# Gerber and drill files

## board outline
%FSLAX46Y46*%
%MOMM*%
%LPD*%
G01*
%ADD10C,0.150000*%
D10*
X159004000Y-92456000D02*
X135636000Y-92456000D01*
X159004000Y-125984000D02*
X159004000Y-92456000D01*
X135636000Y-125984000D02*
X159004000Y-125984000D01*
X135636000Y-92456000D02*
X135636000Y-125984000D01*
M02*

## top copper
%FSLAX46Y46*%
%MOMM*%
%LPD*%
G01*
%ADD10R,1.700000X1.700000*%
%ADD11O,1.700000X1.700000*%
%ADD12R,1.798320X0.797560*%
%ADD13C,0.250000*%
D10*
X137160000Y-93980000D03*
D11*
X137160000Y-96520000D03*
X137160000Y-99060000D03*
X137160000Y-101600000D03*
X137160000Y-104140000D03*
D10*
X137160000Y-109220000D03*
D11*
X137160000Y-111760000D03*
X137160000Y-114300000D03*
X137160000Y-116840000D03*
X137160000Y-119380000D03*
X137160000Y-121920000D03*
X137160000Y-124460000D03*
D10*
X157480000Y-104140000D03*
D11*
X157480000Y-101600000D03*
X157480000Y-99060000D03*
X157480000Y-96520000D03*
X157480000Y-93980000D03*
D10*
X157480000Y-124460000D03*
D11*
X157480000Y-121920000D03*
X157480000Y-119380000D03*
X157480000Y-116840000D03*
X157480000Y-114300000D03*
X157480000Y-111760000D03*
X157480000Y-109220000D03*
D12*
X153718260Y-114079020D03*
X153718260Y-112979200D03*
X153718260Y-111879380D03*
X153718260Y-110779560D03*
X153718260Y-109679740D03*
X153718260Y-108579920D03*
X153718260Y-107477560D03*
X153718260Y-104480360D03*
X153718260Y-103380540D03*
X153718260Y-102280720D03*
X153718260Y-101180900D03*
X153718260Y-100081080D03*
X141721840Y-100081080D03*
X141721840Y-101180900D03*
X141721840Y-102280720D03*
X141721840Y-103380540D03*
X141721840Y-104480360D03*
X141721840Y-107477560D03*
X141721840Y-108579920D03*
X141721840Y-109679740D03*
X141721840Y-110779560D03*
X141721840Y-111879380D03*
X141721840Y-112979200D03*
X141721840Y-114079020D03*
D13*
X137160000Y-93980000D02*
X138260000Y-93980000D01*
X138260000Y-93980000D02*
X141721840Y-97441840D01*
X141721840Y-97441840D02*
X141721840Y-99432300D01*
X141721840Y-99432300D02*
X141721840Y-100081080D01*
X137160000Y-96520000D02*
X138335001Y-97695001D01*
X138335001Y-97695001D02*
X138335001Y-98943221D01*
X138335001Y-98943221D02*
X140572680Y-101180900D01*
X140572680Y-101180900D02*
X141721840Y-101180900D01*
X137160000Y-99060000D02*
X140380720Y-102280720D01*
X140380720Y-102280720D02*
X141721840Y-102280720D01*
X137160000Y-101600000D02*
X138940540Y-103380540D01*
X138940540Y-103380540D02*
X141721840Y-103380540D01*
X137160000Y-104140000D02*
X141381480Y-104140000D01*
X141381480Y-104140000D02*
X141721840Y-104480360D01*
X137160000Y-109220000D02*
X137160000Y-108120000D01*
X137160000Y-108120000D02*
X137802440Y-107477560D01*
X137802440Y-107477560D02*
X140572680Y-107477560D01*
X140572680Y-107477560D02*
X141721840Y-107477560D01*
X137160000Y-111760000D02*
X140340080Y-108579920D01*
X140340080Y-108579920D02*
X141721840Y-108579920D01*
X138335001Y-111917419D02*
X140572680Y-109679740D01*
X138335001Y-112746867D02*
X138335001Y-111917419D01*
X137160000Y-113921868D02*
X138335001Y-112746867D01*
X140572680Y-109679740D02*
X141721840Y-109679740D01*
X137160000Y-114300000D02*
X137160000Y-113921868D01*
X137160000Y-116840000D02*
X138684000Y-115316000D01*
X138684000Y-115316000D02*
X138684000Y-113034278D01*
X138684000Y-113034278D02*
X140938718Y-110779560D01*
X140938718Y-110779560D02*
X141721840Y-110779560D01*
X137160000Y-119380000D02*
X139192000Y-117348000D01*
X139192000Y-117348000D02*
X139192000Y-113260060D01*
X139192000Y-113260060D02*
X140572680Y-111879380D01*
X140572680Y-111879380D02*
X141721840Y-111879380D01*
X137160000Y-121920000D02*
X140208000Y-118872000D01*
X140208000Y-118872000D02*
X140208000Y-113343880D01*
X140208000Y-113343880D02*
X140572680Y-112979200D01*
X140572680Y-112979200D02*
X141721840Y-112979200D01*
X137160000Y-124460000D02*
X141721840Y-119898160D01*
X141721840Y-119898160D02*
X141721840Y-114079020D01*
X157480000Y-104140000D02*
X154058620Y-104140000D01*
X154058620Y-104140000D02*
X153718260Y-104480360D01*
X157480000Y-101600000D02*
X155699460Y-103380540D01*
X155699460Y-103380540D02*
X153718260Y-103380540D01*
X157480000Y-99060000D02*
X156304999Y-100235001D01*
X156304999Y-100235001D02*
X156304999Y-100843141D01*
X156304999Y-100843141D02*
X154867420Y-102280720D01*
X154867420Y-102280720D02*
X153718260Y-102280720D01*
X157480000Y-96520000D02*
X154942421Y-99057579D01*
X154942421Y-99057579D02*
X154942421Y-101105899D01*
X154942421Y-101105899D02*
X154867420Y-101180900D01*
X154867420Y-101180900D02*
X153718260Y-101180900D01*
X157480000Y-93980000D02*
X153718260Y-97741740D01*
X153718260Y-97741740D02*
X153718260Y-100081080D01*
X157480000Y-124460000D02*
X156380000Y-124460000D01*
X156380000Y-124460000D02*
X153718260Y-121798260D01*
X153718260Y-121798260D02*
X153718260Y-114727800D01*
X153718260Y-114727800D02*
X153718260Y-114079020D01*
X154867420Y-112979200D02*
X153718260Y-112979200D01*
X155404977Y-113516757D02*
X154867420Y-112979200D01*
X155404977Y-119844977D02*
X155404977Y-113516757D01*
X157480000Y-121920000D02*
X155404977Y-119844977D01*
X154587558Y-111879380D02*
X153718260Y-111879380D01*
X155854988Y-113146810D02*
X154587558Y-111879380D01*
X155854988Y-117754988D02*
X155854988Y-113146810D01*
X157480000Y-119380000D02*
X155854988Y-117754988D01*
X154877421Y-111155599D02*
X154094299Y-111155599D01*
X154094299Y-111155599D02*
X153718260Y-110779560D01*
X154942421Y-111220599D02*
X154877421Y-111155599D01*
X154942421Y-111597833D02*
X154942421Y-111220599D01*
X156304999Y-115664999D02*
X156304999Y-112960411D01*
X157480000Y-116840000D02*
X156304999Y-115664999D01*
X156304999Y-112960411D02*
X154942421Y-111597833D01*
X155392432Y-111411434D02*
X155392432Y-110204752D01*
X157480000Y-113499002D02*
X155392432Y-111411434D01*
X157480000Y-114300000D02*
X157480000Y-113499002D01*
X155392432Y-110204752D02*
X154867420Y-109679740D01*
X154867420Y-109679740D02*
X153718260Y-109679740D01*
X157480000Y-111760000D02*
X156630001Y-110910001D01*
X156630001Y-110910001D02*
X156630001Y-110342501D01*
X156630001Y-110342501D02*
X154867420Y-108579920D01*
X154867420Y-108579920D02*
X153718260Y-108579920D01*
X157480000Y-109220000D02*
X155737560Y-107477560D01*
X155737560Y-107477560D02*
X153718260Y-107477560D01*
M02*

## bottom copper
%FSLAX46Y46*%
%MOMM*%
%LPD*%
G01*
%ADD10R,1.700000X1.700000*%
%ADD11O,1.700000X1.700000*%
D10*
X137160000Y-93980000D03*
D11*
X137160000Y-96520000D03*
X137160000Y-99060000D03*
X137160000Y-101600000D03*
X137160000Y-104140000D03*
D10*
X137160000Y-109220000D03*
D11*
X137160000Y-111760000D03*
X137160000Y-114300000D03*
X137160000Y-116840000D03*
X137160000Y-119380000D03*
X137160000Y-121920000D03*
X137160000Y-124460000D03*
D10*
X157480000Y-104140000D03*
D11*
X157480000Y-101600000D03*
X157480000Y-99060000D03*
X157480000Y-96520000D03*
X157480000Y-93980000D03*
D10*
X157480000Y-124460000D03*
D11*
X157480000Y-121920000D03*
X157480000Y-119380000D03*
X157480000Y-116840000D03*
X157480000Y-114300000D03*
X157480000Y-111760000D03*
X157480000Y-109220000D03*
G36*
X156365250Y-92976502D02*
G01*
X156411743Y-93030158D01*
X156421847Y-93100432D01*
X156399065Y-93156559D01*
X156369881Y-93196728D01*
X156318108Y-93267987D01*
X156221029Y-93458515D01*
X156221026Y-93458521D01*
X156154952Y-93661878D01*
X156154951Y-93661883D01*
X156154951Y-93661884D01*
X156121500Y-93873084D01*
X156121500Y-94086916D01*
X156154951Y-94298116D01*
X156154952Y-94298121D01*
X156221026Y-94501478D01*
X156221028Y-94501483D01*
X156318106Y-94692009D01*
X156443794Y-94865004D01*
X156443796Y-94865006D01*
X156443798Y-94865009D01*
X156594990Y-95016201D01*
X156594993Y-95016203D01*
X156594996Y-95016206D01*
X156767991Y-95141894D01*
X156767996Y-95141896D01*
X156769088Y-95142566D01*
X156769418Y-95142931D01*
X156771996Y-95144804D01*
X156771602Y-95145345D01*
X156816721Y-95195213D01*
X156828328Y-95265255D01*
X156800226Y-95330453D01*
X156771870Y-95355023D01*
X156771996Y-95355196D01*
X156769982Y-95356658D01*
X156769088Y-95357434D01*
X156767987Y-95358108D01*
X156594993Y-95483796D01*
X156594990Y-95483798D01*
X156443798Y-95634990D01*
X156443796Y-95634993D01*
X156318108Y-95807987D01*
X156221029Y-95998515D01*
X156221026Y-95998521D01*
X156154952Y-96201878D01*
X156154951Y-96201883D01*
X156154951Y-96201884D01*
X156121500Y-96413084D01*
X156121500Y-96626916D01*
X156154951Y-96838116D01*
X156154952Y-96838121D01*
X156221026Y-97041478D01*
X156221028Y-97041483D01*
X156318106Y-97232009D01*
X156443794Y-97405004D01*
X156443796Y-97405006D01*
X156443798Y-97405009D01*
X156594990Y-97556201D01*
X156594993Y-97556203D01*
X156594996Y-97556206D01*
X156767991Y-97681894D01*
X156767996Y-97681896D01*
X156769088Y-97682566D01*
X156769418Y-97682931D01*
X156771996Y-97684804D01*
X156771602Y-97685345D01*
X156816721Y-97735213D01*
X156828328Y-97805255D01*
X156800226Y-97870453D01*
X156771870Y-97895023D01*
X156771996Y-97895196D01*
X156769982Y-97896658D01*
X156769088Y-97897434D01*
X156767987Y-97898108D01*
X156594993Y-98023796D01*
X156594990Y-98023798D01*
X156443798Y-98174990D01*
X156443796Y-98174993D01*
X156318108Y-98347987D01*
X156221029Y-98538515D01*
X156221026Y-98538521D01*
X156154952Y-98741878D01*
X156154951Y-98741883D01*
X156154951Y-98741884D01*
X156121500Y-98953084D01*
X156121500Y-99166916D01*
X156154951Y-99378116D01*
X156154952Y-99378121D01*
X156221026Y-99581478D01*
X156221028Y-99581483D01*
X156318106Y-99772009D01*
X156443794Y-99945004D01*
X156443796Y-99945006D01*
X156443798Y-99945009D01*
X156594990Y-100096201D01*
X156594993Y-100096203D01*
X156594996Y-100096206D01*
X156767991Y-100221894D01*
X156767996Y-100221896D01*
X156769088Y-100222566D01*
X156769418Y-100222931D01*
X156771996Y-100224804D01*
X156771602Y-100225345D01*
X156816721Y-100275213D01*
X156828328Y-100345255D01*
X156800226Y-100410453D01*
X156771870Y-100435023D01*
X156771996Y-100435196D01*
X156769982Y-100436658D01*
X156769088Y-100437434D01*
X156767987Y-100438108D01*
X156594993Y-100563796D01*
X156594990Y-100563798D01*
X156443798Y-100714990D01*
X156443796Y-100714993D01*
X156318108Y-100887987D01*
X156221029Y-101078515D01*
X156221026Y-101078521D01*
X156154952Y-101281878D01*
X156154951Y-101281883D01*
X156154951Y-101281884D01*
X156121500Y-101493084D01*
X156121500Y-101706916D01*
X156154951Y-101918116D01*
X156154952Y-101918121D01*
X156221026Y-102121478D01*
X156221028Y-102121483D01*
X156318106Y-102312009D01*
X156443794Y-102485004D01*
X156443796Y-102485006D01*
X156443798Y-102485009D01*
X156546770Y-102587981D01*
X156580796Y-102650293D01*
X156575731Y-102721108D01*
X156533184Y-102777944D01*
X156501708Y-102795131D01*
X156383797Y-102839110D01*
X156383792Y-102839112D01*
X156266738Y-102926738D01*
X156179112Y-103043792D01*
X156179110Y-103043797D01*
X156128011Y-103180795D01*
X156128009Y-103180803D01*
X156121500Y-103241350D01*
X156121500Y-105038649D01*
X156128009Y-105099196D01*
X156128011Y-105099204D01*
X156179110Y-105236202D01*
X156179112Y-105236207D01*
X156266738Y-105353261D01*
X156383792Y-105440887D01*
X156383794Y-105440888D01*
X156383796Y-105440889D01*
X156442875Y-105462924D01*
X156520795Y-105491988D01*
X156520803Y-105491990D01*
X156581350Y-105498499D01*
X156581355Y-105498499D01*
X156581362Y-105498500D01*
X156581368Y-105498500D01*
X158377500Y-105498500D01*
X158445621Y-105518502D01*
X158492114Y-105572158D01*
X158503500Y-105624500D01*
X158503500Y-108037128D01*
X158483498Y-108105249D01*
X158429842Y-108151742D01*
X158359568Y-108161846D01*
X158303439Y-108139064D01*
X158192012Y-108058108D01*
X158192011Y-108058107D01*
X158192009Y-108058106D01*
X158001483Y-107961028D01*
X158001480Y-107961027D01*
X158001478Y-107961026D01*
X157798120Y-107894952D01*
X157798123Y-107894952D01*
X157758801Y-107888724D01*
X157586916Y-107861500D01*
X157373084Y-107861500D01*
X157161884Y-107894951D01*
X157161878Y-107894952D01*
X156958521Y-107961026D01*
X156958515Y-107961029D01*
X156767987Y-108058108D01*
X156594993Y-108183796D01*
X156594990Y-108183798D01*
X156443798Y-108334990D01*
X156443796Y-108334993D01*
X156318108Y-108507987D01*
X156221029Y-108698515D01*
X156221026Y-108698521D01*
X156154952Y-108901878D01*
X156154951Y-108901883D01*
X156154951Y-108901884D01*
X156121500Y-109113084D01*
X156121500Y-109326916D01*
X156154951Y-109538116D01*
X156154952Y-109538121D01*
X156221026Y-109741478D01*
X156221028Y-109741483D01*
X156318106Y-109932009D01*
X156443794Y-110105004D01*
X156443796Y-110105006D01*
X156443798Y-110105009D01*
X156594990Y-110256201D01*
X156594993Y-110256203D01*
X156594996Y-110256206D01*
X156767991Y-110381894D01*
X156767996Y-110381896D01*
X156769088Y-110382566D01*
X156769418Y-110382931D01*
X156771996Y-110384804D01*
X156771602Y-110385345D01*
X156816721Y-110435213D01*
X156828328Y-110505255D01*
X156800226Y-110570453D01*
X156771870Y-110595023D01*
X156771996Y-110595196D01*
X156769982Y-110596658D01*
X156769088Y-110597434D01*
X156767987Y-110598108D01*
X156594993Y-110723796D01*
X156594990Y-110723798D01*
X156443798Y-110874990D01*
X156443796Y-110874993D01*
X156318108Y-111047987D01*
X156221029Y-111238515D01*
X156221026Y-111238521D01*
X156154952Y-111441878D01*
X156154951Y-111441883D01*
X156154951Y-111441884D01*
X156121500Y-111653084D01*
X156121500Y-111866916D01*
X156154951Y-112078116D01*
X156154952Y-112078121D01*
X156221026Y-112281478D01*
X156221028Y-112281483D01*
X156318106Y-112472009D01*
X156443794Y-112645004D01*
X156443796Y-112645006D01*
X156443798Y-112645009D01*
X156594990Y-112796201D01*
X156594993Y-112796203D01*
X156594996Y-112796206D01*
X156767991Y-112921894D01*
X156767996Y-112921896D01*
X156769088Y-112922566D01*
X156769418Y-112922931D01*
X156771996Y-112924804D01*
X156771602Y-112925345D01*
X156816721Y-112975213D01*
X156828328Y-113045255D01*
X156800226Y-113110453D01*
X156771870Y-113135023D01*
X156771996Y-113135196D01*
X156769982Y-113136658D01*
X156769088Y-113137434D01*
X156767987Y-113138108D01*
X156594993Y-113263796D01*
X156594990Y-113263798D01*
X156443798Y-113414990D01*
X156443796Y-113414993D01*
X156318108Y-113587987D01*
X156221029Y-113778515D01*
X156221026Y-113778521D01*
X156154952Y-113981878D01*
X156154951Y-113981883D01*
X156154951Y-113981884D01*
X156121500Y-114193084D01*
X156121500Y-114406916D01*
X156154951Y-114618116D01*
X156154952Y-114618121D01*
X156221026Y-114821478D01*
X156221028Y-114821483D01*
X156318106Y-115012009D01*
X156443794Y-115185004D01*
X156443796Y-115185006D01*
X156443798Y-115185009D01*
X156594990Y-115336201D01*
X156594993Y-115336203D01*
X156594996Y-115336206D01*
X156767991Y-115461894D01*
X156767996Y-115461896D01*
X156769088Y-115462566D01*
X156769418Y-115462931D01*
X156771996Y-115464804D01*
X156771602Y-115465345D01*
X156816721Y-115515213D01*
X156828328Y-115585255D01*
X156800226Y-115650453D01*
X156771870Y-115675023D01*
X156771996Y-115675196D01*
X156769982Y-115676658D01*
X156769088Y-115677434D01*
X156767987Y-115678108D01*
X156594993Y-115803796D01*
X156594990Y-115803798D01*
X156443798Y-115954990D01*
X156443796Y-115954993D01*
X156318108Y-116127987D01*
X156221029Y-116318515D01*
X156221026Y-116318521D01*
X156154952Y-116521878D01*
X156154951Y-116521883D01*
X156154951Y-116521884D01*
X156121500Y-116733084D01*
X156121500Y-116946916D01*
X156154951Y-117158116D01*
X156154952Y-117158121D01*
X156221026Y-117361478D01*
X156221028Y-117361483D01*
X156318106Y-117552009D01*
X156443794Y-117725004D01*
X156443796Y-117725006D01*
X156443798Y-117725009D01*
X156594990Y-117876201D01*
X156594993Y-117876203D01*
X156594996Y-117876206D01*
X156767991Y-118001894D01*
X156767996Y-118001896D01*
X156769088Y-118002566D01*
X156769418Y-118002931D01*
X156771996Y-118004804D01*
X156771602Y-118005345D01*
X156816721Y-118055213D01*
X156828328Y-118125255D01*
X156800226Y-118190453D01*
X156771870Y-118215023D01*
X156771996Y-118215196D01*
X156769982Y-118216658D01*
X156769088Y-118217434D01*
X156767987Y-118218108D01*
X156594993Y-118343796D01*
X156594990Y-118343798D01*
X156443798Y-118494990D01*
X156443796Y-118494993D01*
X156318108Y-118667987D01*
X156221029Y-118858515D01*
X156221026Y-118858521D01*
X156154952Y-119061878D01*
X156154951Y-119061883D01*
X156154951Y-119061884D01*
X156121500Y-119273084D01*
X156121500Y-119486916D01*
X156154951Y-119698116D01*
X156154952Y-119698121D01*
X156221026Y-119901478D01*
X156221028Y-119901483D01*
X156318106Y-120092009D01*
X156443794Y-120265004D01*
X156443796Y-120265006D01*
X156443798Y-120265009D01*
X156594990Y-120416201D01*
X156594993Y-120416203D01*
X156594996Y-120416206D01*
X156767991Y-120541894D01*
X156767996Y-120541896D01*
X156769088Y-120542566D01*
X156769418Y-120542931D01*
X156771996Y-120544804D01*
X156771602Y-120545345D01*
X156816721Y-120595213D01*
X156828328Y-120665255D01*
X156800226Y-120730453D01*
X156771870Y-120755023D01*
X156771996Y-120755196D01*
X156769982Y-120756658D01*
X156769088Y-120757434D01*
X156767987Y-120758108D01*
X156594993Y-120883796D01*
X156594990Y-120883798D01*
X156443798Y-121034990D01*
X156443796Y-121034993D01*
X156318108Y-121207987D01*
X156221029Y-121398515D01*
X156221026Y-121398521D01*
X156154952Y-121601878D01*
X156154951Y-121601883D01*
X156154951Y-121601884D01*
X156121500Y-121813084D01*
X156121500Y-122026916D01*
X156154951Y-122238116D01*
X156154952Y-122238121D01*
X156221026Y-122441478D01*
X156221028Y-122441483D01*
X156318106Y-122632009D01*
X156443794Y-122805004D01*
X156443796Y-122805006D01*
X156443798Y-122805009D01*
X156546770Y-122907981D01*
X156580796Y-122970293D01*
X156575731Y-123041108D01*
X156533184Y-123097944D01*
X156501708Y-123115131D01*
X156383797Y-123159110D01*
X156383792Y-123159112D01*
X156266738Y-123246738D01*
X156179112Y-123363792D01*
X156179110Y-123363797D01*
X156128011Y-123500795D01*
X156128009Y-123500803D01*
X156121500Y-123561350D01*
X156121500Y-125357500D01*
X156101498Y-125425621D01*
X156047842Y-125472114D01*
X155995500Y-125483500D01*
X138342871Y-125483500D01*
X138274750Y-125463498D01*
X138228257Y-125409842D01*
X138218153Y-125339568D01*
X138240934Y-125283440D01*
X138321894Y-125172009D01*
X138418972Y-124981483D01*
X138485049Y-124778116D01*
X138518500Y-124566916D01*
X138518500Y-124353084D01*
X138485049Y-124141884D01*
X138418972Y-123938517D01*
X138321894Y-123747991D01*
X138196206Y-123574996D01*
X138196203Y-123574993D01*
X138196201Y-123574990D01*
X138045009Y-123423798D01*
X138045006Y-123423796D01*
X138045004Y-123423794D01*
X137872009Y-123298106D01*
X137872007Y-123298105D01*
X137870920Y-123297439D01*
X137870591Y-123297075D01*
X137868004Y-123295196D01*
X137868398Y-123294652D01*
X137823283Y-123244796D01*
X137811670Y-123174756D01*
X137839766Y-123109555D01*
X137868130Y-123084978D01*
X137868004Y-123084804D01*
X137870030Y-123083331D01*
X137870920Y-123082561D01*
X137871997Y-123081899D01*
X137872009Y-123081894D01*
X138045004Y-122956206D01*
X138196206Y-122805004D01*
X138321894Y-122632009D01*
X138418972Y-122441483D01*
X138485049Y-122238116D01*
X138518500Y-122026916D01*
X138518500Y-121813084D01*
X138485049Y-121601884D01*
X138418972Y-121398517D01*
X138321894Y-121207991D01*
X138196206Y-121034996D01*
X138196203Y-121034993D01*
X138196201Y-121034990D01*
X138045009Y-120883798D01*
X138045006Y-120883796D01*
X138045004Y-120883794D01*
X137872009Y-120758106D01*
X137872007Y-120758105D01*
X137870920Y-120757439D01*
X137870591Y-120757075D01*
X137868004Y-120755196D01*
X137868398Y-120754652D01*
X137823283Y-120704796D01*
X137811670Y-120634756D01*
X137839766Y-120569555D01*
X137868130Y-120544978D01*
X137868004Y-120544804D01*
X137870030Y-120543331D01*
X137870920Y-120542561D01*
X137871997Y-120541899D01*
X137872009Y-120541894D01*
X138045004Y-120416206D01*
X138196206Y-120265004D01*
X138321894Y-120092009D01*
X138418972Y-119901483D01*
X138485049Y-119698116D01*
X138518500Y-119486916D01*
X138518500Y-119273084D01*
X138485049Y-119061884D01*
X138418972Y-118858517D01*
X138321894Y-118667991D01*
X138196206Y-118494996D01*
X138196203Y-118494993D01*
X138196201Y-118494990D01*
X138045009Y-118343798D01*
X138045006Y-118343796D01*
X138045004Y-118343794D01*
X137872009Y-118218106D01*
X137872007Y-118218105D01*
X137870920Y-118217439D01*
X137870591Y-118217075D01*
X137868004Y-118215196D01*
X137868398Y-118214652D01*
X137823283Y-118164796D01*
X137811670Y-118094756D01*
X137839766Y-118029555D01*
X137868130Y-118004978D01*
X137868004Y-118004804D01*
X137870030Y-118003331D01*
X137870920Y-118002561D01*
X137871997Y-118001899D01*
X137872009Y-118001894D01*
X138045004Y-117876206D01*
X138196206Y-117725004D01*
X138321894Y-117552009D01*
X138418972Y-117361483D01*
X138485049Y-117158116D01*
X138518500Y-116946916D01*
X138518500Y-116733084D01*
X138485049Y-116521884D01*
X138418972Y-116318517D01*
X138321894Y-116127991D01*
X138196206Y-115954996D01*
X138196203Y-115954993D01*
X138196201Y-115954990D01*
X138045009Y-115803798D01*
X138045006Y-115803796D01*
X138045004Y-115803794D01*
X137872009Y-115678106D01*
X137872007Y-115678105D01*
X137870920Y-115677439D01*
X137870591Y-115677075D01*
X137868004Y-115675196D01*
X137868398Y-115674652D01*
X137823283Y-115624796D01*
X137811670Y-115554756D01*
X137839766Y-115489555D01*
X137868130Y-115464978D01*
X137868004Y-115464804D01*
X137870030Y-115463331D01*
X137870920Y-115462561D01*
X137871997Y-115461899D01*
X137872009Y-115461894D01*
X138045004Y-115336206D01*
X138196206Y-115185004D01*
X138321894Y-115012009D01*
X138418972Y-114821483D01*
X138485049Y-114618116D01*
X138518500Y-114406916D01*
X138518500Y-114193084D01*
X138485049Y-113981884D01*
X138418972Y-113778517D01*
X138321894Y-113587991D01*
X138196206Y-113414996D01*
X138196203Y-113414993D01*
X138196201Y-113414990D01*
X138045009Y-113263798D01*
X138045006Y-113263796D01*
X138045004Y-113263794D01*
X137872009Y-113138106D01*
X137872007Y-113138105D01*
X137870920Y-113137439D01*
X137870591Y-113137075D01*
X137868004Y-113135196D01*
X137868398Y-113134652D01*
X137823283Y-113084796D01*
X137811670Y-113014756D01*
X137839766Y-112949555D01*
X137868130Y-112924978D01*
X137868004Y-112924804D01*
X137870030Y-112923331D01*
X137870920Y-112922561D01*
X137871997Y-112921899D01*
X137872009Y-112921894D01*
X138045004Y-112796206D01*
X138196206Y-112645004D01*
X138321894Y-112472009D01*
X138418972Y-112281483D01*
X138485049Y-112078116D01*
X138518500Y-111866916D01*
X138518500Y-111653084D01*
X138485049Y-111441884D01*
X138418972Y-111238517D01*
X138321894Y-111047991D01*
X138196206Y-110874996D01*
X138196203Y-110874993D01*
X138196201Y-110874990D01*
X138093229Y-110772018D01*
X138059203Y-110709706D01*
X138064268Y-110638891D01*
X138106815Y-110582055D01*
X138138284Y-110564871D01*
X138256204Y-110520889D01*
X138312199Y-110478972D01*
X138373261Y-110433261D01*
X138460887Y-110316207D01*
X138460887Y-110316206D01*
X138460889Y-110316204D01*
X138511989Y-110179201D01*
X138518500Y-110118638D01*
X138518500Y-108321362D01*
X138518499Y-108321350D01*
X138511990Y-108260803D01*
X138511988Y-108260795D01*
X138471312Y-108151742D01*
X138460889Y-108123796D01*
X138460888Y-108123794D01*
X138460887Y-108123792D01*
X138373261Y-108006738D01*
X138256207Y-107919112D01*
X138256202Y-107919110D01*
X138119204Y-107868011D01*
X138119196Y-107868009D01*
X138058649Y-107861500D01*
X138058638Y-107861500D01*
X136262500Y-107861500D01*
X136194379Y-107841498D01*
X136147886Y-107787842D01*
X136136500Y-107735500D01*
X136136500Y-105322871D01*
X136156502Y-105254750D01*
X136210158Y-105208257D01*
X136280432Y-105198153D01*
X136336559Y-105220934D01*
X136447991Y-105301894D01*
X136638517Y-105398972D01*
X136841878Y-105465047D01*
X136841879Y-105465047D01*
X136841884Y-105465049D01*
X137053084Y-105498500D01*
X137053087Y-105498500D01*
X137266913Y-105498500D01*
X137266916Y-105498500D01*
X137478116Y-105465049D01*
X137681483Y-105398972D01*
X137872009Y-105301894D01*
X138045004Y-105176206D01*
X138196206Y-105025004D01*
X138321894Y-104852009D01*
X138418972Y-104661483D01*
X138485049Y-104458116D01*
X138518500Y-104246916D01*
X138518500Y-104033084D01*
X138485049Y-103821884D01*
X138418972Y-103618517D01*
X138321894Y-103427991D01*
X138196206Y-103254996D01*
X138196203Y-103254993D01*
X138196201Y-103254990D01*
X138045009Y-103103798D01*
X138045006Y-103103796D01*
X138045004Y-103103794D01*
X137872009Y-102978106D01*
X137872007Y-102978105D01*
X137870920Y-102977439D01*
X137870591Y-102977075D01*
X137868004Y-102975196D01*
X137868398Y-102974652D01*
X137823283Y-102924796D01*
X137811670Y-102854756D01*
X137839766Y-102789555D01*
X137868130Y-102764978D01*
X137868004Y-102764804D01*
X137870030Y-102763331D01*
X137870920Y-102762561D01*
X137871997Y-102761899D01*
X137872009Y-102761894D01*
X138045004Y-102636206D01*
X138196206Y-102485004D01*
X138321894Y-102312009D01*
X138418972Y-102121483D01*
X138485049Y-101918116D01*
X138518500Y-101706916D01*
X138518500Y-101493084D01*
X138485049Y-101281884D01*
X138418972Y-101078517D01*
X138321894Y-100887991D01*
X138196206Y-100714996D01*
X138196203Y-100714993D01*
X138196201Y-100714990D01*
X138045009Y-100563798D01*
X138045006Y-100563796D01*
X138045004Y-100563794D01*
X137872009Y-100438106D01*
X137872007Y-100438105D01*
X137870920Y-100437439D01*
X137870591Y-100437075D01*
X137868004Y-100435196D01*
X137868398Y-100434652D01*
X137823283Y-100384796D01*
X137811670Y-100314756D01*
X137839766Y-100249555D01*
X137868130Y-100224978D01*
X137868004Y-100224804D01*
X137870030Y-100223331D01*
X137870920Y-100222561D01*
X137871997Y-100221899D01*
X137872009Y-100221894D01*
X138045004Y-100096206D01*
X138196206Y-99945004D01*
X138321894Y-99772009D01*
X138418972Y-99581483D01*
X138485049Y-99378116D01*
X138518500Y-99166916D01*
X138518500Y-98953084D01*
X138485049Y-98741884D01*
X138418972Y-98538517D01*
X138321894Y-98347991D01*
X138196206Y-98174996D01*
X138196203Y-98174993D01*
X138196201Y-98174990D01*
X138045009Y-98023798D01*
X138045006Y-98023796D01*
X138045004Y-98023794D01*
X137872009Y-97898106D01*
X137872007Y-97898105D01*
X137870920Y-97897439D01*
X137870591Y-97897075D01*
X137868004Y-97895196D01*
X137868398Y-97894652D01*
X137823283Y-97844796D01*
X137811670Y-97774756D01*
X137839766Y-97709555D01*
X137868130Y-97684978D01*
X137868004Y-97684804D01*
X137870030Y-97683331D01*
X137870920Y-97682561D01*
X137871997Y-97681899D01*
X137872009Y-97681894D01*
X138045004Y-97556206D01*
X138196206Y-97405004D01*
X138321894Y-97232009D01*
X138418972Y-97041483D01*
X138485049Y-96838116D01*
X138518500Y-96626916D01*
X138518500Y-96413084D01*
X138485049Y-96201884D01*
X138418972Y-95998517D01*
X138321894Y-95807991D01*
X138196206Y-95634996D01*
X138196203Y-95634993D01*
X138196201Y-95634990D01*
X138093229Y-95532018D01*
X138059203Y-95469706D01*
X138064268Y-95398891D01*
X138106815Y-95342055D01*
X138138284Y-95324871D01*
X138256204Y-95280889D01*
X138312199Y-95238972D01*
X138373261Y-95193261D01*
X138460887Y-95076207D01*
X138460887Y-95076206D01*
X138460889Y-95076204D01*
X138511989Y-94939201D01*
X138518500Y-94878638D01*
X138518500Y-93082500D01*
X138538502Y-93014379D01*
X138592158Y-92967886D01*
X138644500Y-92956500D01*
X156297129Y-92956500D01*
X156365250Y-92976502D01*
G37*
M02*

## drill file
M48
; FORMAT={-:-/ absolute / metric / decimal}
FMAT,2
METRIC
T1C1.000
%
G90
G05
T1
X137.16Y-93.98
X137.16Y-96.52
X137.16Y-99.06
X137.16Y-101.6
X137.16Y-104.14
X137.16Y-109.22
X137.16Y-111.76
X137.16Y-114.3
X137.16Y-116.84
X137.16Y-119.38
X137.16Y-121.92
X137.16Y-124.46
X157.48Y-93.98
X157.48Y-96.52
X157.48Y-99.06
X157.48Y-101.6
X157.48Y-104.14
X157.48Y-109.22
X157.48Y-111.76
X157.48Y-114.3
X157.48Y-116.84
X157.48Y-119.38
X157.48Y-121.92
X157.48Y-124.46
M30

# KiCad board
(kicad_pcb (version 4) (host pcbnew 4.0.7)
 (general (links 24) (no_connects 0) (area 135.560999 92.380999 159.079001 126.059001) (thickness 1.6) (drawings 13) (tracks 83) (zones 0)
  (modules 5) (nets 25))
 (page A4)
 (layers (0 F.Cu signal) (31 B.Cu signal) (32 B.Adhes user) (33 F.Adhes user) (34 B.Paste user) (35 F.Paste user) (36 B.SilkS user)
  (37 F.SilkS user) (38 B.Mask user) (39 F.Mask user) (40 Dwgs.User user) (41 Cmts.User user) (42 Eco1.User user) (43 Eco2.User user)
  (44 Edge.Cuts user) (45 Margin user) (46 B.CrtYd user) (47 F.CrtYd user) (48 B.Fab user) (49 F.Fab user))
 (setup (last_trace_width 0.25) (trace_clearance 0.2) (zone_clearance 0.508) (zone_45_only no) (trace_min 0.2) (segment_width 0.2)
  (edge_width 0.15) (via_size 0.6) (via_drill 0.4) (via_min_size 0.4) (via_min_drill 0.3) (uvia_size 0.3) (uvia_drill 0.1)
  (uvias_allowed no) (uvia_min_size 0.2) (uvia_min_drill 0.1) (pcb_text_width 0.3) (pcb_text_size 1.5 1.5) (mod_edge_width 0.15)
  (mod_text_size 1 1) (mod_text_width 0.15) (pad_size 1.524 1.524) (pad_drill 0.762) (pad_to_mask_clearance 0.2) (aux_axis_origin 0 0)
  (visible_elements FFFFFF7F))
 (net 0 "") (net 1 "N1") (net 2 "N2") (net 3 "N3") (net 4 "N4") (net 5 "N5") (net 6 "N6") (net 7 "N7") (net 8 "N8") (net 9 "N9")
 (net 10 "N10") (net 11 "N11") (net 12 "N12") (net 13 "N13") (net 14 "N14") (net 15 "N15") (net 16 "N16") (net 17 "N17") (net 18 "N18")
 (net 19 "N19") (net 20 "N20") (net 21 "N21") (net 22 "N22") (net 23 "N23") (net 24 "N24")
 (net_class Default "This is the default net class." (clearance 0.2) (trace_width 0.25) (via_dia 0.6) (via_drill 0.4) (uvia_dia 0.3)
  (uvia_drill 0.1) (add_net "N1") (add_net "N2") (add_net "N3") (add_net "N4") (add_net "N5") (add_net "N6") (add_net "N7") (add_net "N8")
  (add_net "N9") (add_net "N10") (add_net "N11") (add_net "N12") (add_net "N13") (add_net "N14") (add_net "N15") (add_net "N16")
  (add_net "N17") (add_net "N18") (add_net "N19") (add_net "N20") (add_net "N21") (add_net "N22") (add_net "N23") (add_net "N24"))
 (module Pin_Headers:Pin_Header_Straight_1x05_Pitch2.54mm (layer F.Cu) (at 137.16 93.98)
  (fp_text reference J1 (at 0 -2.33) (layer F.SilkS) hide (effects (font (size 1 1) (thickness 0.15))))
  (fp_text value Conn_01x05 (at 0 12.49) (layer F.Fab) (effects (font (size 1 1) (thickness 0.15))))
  (pad 1 thru_hole rect (at 0 0) (size 1.7 1.7) (drill 1) (layers *.Cu *.Mask) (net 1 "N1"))
  (pad 2 thru_hole oval (at 0 2.54) (size 1.7 1.7) (drill 1) (layers *.Cu *.Mask) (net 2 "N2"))
  (pad 3 thru_hole oval (at 0 5.08) (size 1.7 1.7) (drill 1) (layers *.Cu *.Mask) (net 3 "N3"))
  (pad 4 thru_hole oval (at 0 7.62) (size 1.7 1.7) (drill 1) (layers *.Cu *.Mask) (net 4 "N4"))
  (pad 5 thru_hole oval (at 0 10.16) (size 1.7 1.7) (drill 1) (layers *.Cu *.Mask) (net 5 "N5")))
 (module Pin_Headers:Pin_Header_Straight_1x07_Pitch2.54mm (layer F.Cu) (at 137.16 109.22)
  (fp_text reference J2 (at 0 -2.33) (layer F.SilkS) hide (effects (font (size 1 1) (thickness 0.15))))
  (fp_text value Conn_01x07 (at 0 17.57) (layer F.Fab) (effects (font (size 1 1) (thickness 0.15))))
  (pad 1 thru_hole rect (at 0 0) (size 1.7 1.7) (drill 1) (layers *.Cu *.Mask) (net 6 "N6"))
  (pad 2 thru_hole oval (at 0 2.54) (size 1.7 1.7) (drill 1) (layers *.Cu *.Mask) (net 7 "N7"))
  (pad 3 thru_hole oval (at 0 5.08) (size 1.7 1.7) (drill 1) (layers *.Cu *.Mask) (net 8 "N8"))
  (pad 4 thru_hole oval (at 0 7.62) (size 1.7 1.7) (drill 1) (layers *.Cu *.Mask) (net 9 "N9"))
  (pad 5 thru_hole oval (at 0 10.16) (size 1.7 1.7) (drill 1) (layers *.Cu *.Mask) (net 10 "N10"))
  (pad 6 thru_hole oval (at 0 12.7) (size 1.7 1.7) (drill 1) (layers *.Cu *.Mask) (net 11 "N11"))
  (pad 7 thru_hole oval (at 0 15.24) (size 1.7 1.7) (drill 1) (layers *.Cu *.Mask) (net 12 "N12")))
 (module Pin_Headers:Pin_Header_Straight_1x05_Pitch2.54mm (layer F.Cu) (at 157.48 104.14 180)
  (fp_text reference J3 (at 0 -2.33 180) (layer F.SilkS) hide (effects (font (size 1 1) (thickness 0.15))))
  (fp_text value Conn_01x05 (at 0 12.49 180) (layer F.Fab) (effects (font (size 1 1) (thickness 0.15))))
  (pad 1 thru_hole rect (at 0 0 180) (size 1.7 1.7) (drill 1) (layers *.Cu *.Mask) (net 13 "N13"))
  (pad 2 thru_hole oval (at 0 2.54 180) (size 1.7 1.7) (drill 1) (layers *.Cu *.Mask) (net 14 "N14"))
  (pad 3 thru_hole oval (at 0 5.08 180) (size 1.7 1.7) (drill 1) (layers *.Cu *.Mask) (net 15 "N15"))
  (pad 4 thru_hole oval (at 0 7.62 180) (size 1.7 1.7) (drill 1) (layers *.Cu *.Mask) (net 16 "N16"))
  (pad 5 thru_hole oval (at 0 10.16 180) (size 1.7 1.7) (drill 1) (layers *.Cu *.Mask) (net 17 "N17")))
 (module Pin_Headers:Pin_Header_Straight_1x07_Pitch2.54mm (layer F.Cu) (at 157.48 124.46 180)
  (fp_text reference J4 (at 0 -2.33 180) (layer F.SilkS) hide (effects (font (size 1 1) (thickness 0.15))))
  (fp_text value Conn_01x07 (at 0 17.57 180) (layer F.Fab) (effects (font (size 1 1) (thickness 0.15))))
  (pad 1 thru_hole rect (at 0 0 180) (size 1.7 1.7) (drill 1) (layers *.Cu *.Mask) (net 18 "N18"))
  (pad 2 thru_hole oval (at 0 2.54 180) (size 1.7 1.7) (drill 1) (layers *.Cu *.Mask) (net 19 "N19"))
  (pad 3 thru_hole oval (at 0 5.08 180) (size 1.7 1.7) (drill 1) (layers *.Cu *.Mask) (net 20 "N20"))
  (pad 4 thru_hole oval (at 0 7.62 180) (size 1.7 1.7) (drill 1) (layers *.Cu *.Mask) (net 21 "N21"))
  (pad 5 thru_hole oval (at 0 10.16 180) (size 1.7 1.7) (drill 1) (layers *.Cu *.Mask) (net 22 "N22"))
  (pad 6 thru_hole oval (at 0 12.7 180) (size 1.7 1.7) (drill 1) (layers *.Cu *.Mask) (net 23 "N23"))
  (pad 7 thru_hole oval (at 0 15.24 180) (size 1.7 1.7) (drill 1) (layers *.Cu *.Mask) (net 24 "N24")))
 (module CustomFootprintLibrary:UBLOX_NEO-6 (layer F.Cu) (at 147.32 106.68)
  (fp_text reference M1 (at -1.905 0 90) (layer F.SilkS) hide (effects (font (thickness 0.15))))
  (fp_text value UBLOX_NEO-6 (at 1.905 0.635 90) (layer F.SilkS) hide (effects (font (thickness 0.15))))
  (pad 1_RE smd rect (at 6.39826 7.39902 90) (size 0.79756 1.79832) (layers F.Cu F.Paste F.Mask) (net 18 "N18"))
  (pad 2_SS smd rect (at 6.39826 6.2992 90) (size 0.79756 1.79832) (layers F.Cu F.Paste F.Mask) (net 19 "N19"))
  (pad 3_TI smd rect (at 6.39826 5.19938 90) (size 0.79756 1.79832) (layers F.Cu F.Paste F.Mask) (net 20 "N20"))
  (pad 4_EX smd rect (at 6.39826 4.09956 90) (size 0.79756 1.79832) (layers F.Cu F.Paste F.Mask) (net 21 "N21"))
  (pad 5_US smd rect (at 6.39826 2.99974 90) (size 0.79756 1.79832) (layers F.Cu F.Paste F.Mask) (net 22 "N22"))
  (pad 6_US smd rect (at 6.39826 1.89992 90) (size 0.79756 1.79832) (layers F.Cu F.Paste F.Mask) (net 23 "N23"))
  (pad 7_VD smd rect (at 6.39826 0.79756 90) (size 0.79756 1.79832) (layers F.Cu F.Paste F.Mask) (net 24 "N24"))
  (pad 8_RE smd rect (at 6.39826 -2.19964 90) (size 0.79756 1.79832) (layers F.Cu F.Paste F.Mask) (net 13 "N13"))
  (pad 9_VC smd rect (at 6.39826 -3.29946 90) (size 0.79756 1.79832) (layers F.Cu F.Paste F.Mask) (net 14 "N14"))
  (pad 10_G smd rect (at 6.39826 -4.39928 90) (size 0.79756 1.79832) (layers F.Cu F.Paste F.Mask) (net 15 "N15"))
  (pad 11_R smd rect (at 6.39826 -5.4991 90) (size 0.79756 1.79832) (layers F.Cu F.Paste F.Mask) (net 16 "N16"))
  (pad 12_G smd rect (at 6.39826 -6.59892 90) (size 0.79756 1.79832) (layers F.Cu F.Paste F.Mask) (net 17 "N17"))
  (pad 13_G smd rect (at -5.59816 -6.59892 90) (size 0.79756 1.79832) (layers F.Cu F.Paste F.Mask) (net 1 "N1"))
  (pad 14_M smd rect (at -5.59816 -5.4991 90) (size 0.79756 1.79832) (layers F.Cu F.Paste F.Mask) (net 2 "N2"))
  (pad 15_M smd rect (at -5.59816 -4.39928 90) (size 0.79756 1.79832) (layers F.Cu F.Paste F.Mask) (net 3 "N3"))
  (pad 16_C smd rect (at -5.59816 -3.29946 90) (size 0.79756 1.79832) (layers F.Cu F.Paste F.Mask) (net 4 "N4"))
  (pad 17_R smd rect (at -5.59816 -2.19964 90) (size 0.79756 1.79832) (layers F.Cu F.Paste F.Mask) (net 5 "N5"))
  (pad 18_S smd rect (at -5.59816 0.79756 90) (size 0.79756 1.79832) (layers F.Cu F.Paste F.Mask) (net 6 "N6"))
  (pad 19_S smd rect (at -5.59816 1.89992 90) (size 0.79756 1.79832) (layers F.Cu F.Paste F.Mask) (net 7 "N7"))
  (pad 20_T smd rect (at -5.59816 2.99974 90) (size 0.79756 1.79832) (layers F.Cu F.Paste F.Mask) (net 8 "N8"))
  (pad 21_R smd rect (at -5.59816 4.09956 90) (size 0.79756 1.79832) (layers F.Cu F.Paste F.Mask) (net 9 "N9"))
  (pad 22_V smd rect (at -5.59816 5.19938 90) (size 0.79756 1.79832) (layers F.Cu F.Paste F.Mask) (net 10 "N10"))
  (pad 23_V smd rect (at -5.59816 6.2992 90) (size 0.79756 1.79832) (layers F.Cu F.Paste F.Mask) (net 11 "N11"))
  (pad 24_G smd rect (at -5.59816 7.39902 90) (size 0.79756 1.79832) (layers F.Cu F.Paste F.Mask) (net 12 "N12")))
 (gr_line (start 159.004 92.456) (end 135.636 92.456) (layer Edge.Cuts) (width 0.15))
 (gr_line (start 159.004 125.984) (end 159.004 92.456) (layer Edge.Cuts) (width 0.15))
 (gr_line (start 135.636 125.984) (end 159.004 125.984) (layer Edge.Cuts) (width 0.15))
 (gr_line (start 135.636 92.456) (end 135.636 125.984) (layer Edge.Cuts) (width 0.15))
 (segment (start 137.16 93.98) (end 138.26 93.98) (width 0.25) (layer F.Cu) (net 1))
 (segment (start 138.26 93.98) (end 141.72184 97.44184) (width 0.25) (layer F.Cu) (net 1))
 (segment (start 141.72184 97.44184) (end 141.72184 99.4323) (width 0.25) (layer F.Cu) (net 1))
 (segment (start 141.72184 99.4323) (end 141.72184 100.08108) (width 0.25) (layer F.Cu) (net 1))
 (segment (start 137.16 96.52) (end 138.335001 97.695001) (width 0.25) (layer F.Cu) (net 2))
 (segment (start 138.335001 97.695001) (end 138.335001 98.943221) (width 0.25) (layer F.Cu) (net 2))
 (segment (start 138.335001 98.943221) (end 140.57268 101.1809) (width 0.25) (layer F.Cu) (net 2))
 (segment (start 140.57268 101.1809) (end 141.72184 101.1809) (width 0.25) (layer F.Cu) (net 2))
 (segment (start 137.16 99.06) (end 140.38072 102.28072) (width 0.25) (layer F.Cu) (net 3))
 (segment (start 140.38072 102.28072) (end 141.72184 102.28072) (width 0.25) (layer F.Cu) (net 3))
 (segment (start 137.16 101.6) (end 138.94054 103.38054) (width 0.25) (layer F.Cu) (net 4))
 (segment (start 138.94054 103.38054) (end 141.72184 103.38054) (width 0.25) (layer F.Cu) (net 4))
 (segment (start 137.16 104.14) (end 141.38148 104.14) (width 0.25) (layer F.Cu) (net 5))
 (segment (start 141.38148 104.14) (end 141.72184 104.48036) (width 0.25) (layer F.Cu) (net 5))
 (segment (start 137.16 109.22) (end 137.16 108.12) (width 0.25) (layer F.Cu) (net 6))
 (segment (start 137.16 108.12) (end 137.80244 107.47756) (width 0.25) (layer F.Cu) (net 6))
 (segment (start 137.80244 107.47756) (end 140.57268 107.47756) (width 0.25) (layer F.Cu) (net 6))
 (segment (start 140.57268 107.47756) (end 141.72184 107.47756) (width 0.25) (layer F.Cu) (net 6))
 (segment (start 137.16 111.76) (end 140.34008 108.57992) (width 0.25) (layer F.Cu) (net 7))
 (segment (start 140.34008 108.57992) (end 141.72184 108.57992) (width 0.25) (layer F.Cu) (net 7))
 (segment (start 138.335001 111.917419) (end 140.57268 109.67974) (width 0.25) (layer F.Cu) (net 8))
 (segment (start 138.335001 112.746867) (end 138.335001 111.917419) (width 0.25) (layer F.Cu) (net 8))
 (segment (start 137.16 113.921868) (end 138.335001 112.746867) (width 0.25) (layer F.Cu) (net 8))
 (segment (start 140.57268 109.67974) (end 141.72184 109.67974) (width 0.25) (layer F.Cu) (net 8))
 (segment (start 137.16 114.3) (end 137.16 113.921868) (width 0.25) (layer F.Cu) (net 8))
 (segment (start 137.16 116.84) (end 138.684 115.316) (width 0.25) (layer F.Cu) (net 9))
 (segment (start 138.684 115.316) (end 138.684 113.034278) (width 0.25) (layer F.Cu) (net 9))
 (segment (start 138.684 113.034278) (end 140.938718 110.77956) (width 0.25) (layer F.Cu) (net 9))
 (segment (start 140.938718 110.77956) (end 141.72184 110.77956) (width 0.25) (layer F.Cu) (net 9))
 (segment (start 137.16 119.38) (end 139.192 117.348) (width 0.25) (layer F.Cu) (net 10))
 (segment (start 139.192 117.348) (end 139.192 113.26006) (width 0.25) (layer F.Cu) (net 10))
 (segment (start 139.192 113.26006) (end 140.57268 111.87938) (width 0.25) (layer F.Cu) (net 10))
 (segment (start 140.57268 111.87938) (end 141.72184 111.87938) (width 0.25) (layer F.Cu) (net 10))
 (segment (start 137.16 121.92) (end 140.208 118.872) (width 0.25) (layer F.Cu) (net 11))
 (segment (start 140.208 118.872) (end 140.208 113.34388) (width 0.25) (layer F.Cu) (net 11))
 (segment (start 140.208 113.34388) (end 140.57268 112.9792) (width 0.25) (layer F.Cu) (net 11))
 (segment (start 140.57268 112.9792) (end 141.72184 112.9792) (width 0.25) (layer F.Cu) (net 11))
 (segment (start 137.16 124.46) (end 141.72184 119.89816) (width 0.25) (layer F.Cu) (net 12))
 (segment (start 141.72184 119.89816) (end 141.72184 114.07902) (width 0.25) (layer F.Cu) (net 12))
 (segment (start 157.48 104.14) (end 154.05862 104.14) (width 0.25) (layer F.Cu) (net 13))
 (segment (start 154.05862 104.14) (end 153.71826 104.48036) (width 0.25) (layer F.Cu) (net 13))
 (segment (start 157.48 101.6) (end 155.69946 103.38054) (width 0.25) (layer F.Cu) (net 14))
 (segment (start 155.69946 103.38054) (end 153.71826 103.38054) (width 0.25) (layer F.Cu) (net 14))
 (segment (start 157.48 99.06) (end 156.304999 100.235001) (width 0.25) (layer F.Cu) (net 15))
 (segment (start 156.304999 100.235001) (end 156.304999 100.843141) (width 0.25) (layer F.Cu) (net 15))
 (segment (start 156.304999 100.843141) (end 154.86742 102.28072) (width 0.25) (layer F.Cu) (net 15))
 (segment (start 154.86742 102.28072) (end 153.71826 102.28072) (width 0.25) (layer F.Cu) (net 15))
 (segment (start 157.48 96.52) (end 154.942421 99.057579) (width 0.25) (layer F.Cu) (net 16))
 (segment (start 154.942421 99.057579) (end 154.942421 101.105899) (width 0.25) (layer F.Cu) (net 16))
 (segment (start 154.942421 101.105899) (end 154.86742 101.1809) (width 0.25) (layer F.Cu) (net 16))
 (segment (start 154.86742 101.1809) (end 153.71826 101.1809) (width 0.25) (layer F.Cu) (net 16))
 (segment (start 157.48 93.98) (end 153.71826 97.74174) (width 0.25) (layer F.Cu) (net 17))
 (segment (start 153.71826 97.74174) (end 153.71826 100.08108) (width 0.25) (layer F.Cu) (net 17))
 (segment (start 157.48 124.46) (end 156.38 124.46) (width 0.25) (layer F.Cu) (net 18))
 (segment (start 156.38 124.46) (end 153.71826 121.79826) (width 0.25) (layer F.Cu) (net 18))
 (segment (start 153.71826 121.79826) (end 153.71826 114.7278) (width 0.25) (layer F.Cu) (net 18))
 (segment (start 153.71826 114.7278) (end 153.71826 114.07902) (width 0.25) (layer F.Cu) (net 18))
 (segment (start 154.86742 112.9792) (end 153.71826 112.9792) (width 0.25) (layer F.Cu) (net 19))
 (segment (start 155.404977 113.516757) (end 154.86742 112.9792) (width 0.25) (layer F.Cu) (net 19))
 (segment (start 155.404977 119.844977) (end 155.404977 113.516757) (width 0.25) (layer F.Cu) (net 19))
 (segment (start 157.48 121.92) (end 155.404977 119.844977) (width 0.25) (layer F.Cu) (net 19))
 (segment (start 154.587558 111.87938) (end 153.71826 111.87938) (width 0.25) (layer F.Cu) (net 20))
 (segment (start 155.854988 113.14681) (end 154.587558 111.87938) (width 0.25) (layer F.Cu) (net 20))
 (segment (start 155.854988 117.754988) (end 155.854988 113.14681) (width 0.25) (layer F.Cu) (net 20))
 (segment (start 157.48 119.38) (end 155.854988 117.754988) (width 0.25) (layer F.Cu) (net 20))
 (segment (start 154.877421 111.155599) (end 154.094299 111.155599) (width 0.25) (layer F.Cu) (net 21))
 (segment (start 154.094299 111.155599) (end 153.71826 110.77956) (width 0.25) (layer F.Cu) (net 21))
 (segment (start 154.942421 111.220599) (end 154.877421 111.155599) (width 0.25) (layer F.Cu) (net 21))
 (segment (start 154.942421 111.597833) (end 154.942421 111.220599) (width 0.25) (layer F.Cu) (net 21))
 (segment (start 156.304999 115.664999) (end 156.304999 112.960411) (width 0.25) (layer F.Cu) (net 21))
 (segment (start 157.48 116.84) (end 156.304999 115.664999) (width 0.25) (layer F.Cu) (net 21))
 (segment (start 156.304999 112.960411) (end 154.942421 111.597833) (width 0.25) (layer F.Cu) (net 21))
 (segment (start 155.392432 111.411434) (end 155.392432 110.204752) (width 0.25) (layer F.Cu) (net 22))
 (segment (start 157.48 113.499002) (end 155.392432 111.411434) (width 0.25) (layer F.Cu) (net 22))
 (segment (start 157.48 114.3) (end 157.48 113.499002) (width 0.25) (layer F.Cu) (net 22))
 (segment (start 155.392432 110.204752) (end 154.86742 109.67974) (width 0.25) (layer F.Cu) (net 22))
 (segment (start 154.86742 109.67974) (end 153.71826 109.67974) (width 0.25) (layer F.Cu) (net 22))
 (segment (start 157.48 111.76) (end 156.630001 110.910001) (width 0.25) (layer F.Cu) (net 23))
 (segment (start 156.630001 110.910001) (end 156.630001 110.342501) (width 0.25) (layer F.Cu) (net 23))
 (segment (start 156.630001 110.342501) (end 154.86742 108.57992) (width 0.25) (layer F.Cu) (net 23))
 (segment (start 154.86742 108.57992) (end 153.71826 108.57992) (width 0.25) (layer F.Cu) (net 23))
 (segment (start 157.48 109.22) (end 155.73756 107.47756) (width 0.25) (layer F.Cu) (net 24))
 (segment (start 155.73756 107.47756) (end 153.71826 107.47756) (width 0.25) (layer F.Cu) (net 24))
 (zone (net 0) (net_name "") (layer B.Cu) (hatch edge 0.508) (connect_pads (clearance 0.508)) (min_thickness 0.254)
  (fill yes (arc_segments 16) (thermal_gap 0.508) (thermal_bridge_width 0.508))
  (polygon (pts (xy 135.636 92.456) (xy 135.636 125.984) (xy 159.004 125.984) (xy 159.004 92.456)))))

